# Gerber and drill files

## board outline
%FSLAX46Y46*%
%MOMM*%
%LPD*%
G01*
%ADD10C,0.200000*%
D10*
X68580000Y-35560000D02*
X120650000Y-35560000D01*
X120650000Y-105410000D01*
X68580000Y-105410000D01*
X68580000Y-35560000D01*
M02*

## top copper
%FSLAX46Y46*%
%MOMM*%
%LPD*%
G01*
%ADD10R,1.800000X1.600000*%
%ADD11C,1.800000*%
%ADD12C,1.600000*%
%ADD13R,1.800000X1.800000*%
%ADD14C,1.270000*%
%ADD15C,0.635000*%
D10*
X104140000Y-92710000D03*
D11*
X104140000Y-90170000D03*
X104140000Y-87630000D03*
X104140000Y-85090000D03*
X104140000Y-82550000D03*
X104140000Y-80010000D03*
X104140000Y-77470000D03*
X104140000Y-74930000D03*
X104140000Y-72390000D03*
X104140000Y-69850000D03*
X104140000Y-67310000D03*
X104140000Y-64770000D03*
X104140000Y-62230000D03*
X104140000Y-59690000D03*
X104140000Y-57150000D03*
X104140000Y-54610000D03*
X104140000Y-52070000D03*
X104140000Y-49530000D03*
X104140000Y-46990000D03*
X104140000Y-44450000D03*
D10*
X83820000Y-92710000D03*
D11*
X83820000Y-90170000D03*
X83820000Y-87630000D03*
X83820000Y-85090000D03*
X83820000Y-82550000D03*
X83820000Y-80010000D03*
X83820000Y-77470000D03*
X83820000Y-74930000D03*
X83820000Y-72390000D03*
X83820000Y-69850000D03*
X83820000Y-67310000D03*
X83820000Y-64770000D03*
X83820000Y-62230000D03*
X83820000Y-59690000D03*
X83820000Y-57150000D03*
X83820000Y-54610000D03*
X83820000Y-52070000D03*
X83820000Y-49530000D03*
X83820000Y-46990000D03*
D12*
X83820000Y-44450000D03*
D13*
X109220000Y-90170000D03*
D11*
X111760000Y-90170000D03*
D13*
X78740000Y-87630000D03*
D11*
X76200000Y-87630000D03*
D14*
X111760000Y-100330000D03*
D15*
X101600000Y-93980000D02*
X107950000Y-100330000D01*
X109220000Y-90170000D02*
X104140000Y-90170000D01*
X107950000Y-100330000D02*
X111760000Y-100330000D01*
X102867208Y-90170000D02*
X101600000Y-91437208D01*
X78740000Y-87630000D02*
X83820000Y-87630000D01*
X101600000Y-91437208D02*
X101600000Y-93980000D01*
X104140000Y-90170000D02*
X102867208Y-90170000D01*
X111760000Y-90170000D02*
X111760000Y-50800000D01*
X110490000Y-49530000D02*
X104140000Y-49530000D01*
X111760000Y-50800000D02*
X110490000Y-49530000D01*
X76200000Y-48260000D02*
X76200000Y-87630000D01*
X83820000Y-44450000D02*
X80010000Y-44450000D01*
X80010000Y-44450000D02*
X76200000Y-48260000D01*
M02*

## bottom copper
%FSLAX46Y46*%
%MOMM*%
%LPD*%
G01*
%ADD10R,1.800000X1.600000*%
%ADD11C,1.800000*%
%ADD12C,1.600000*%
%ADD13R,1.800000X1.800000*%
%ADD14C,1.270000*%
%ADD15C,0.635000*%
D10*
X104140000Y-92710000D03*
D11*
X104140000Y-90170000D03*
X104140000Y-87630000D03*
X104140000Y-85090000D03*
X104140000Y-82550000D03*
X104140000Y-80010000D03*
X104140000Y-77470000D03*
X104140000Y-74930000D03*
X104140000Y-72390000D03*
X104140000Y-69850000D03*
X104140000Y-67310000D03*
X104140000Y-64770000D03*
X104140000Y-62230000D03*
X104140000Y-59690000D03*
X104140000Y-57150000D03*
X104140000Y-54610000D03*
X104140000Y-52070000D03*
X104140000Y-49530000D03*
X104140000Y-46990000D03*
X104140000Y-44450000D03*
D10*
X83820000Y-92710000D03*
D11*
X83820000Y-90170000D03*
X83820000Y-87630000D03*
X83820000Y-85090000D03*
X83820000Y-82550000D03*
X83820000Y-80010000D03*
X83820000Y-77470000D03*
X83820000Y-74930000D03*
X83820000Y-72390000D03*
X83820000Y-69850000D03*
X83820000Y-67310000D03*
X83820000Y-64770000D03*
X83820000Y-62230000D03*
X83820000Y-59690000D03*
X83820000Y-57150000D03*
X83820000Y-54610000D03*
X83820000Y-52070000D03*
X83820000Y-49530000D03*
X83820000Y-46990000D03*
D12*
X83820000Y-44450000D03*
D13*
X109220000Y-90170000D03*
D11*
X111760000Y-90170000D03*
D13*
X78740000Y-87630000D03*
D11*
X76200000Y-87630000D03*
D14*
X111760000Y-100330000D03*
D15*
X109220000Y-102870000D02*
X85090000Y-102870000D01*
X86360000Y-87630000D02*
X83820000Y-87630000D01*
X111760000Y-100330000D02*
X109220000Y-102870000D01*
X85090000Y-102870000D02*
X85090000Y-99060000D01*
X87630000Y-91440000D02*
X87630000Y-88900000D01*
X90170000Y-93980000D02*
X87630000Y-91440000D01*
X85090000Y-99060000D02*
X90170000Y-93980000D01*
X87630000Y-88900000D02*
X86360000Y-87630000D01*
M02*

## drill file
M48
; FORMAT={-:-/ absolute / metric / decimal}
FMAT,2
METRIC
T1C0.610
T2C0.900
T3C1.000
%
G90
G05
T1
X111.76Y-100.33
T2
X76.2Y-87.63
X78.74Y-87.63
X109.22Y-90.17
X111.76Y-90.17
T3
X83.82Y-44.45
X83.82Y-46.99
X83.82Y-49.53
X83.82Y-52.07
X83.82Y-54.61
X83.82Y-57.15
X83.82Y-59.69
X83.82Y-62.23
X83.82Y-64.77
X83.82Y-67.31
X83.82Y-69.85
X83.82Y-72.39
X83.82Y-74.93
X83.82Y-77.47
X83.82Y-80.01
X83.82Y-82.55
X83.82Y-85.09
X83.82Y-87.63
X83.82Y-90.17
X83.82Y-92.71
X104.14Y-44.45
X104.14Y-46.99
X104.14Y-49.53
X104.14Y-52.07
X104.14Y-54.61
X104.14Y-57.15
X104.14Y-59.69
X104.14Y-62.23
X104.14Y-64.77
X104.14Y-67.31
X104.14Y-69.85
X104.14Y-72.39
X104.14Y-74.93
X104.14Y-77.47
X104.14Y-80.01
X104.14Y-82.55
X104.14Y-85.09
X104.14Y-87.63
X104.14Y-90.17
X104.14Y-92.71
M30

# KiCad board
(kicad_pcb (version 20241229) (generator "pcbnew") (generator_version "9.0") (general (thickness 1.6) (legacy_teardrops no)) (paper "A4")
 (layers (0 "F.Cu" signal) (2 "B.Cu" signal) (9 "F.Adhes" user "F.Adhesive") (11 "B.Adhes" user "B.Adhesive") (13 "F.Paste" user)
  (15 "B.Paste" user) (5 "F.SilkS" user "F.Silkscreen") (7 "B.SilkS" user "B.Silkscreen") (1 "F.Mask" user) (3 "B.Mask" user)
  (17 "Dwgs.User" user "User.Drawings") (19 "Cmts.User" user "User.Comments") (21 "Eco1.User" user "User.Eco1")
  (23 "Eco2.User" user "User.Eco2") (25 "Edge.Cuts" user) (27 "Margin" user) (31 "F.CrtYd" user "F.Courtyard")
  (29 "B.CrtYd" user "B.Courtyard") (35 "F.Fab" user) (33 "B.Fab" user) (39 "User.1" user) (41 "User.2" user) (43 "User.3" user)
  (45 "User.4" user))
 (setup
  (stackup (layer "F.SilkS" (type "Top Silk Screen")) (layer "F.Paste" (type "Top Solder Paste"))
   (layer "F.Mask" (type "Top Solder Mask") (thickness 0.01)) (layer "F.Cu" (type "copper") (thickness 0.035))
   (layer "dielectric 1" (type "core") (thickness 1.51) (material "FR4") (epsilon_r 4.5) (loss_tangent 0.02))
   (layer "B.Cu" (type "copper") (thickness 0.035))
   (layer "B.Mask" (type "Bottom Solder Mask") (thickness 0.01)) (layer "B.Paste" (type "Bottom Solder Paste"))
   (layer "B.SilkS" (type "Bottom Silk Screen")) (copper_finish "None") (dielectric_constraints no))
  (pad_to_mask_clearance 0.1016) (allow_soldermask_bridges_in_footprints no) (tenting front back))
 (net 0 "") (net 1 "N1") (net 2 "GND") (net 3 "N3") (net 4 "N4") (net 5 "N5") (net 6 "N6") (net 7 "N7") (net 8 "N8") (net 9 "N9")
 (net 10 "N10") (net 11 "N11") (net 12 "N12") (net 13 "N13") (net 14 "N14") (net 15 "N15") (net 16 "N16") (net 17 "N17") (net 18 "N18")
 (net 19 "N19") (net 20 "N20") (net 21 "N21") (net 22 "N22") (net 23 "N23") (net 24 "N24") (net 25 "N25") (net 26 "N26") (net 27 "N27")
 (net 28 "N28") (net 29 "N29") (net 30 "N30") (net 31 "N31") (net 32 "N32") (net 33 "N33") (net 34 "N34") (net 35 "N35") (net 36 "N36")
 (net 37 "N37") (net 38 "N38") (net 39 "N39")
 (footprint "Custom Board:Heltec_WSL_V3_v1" (layer "F.Cu") (at 93.98 72.39)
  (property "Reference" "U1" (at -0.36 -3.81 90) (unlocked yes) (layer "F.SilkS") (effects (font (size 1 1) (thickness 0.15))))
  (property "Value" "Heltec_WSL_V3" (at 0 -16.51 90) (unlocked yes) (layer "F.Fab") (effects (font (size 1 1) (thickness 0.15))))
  (pad "1" thru_hole rect (at 10.16 20.32) (size 1.8 1.6) (drill 1) (layers "*.Cu" "*.Mask") (remove_unused_layers no) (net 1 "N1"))
  (pad "2" thru_hole circle (at 10.16 17.78 270) (size 1.8 1.8) (drill 1) (layers "*.Cu" "*.Mask") (remove_unused_layers no) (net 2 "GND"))
  (pad "3" thru_hole circle (at 10.16 15.24 270) (size 1.8 1.8) (drill 1) (layers "*.Cu" "*.Mask") (remove_unused_layers no) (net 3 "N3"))
  (pad "4" thru_hole circle (at 10.16 12.7 270) (size 1.8 1.8) (drill 1) (layers "*.Cu" "*.Mask") (remove_unused_layers no) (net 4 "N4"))
  (pad "5" thru_hole circle (at 10.16 10.16 270) (size 1.8 1.8) (drill 1) (layers "*.Cu" "*.Mask") (remove_unused_layers no) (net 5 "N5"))
  (pad "6" thru_hole circle (at 10.16 7.62 270) (size 1.8 1.8) (drill 1) (layers "*.Cu" "*.Mask") (remove_unused_layers no) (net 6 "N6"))
  (pad "7" thru_hole circle (at 10.16 5.08 270) (size 1.8 1.8) (drill 1) (layers "*.Cu" "*.Mask") (remove_unused_layers no) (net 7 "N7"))
  (pad "8" thru_hole circle (at 10.16 2.54 270) (size 1.8 1.8) (drill 1) (layers "*.Cu" "*.Mask") (remove_unused_layers no) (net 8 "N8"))
  (pad "9" thru_hole circle (at 10.16 0 270) (size 1.8 1.8) (drill 1) (layers "*.Cu" "*.Mask") (remove_unused_layers no) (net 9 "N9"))
  (pad "10" thru_hole circle (at 10.16 -2.54 270) (size 1.8 1.8) (drill 1) (layers "*.Cu" "*.Mask") (remove_unused_layers no) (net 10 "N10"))
  (pad "11" thru_hole circle (at 10.16 -5.08 270) (size 1.8 1.8) (drill 1) (layers "*.Cu" "*.Mask") (remove_unused_layers no) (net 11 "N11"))
  (pad "12" thru_hole circle (at 10.16 -7.62 270) (size 1.8 1.8) (drill 1) (layers "*.Cu" "*.Mask") (remove_unused_layers no) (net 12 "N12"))
  (pad "13" thru_hole circle (at 10.16 -10.16 270) (size 1.8 1.8) (drill 1) (layers "*.Cu" "*.Mask") (remove_unused_layers no)
   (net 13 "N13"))
  (pad "14" thru_hole circle (at 10.16 -12.7 270) (size 1.8 1.8) (drill 1) (layers "*.Cu" "*.Mask") (remove_unused_layers no) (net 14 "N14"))
  (pad "15" thru_hole circle (at 10.16 -15.24 270) (size 1.8 1.8) (drill 1) (layers "*.Cu" "*.Mask") (remove_unused_layers no)
   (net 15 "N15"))
  (pad "16" thru_hole circle (at 10.16 -17.78 270) (size 1.8 1.8) (drill 1) (layers "*.Cu" "*.Mask") (remove_unused_layers no)
   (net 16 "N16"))
  (pad "17" thru_hole circle (at 10.16 -20.32 270) (size 1.8 1.8) (drill 1) (layers "*.Cu" "*.Mask") (remove_unused_layers no)
   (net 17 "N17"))
  (pad "18" thru_hole circle (at 10.16 -22.86 270) (size 1.8 1.8) (drill 1) (layers "*.Cu" "*.Mask") (remove_unused_layers no)
   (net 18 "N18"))
  (pad "19" thru_hole circle (at 10.16 -25.4 270) (size 1.8 1.8) (drill 1) (layers "*.Cu" "*.Mask") (remove_unused_layers no) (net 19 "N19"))
  (pad "20" thru_hole circle (at 10.16 -27.94 270) (size 1.8 1.8) (drill 1) (layers "*.Cu" "*.Mask") (remove_unused_layers no)
   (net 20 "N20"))
  (pad "21" thru_hole rect (at -10.16 20.32) (size 1.8 1.6) (drill 1) (layers "*.Cu" "*.Mask") (remove_unused_layers no) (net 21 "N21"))
  (pad "22" thru_hole circle (at -10.16 17.78 270) (size 1.8 1.8) (drill 1) (layers "*.Cu" "*.Mask") (remove_unused_layers no)
   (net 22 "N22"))
  (pad "23" thru_hole circle (at -10.16 15.24 270) (size 1.8 1.8) (drill 1) (layers "*.Cu" "*.Mask") (remove_unused_layers no) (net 2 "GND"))
  (pad "24" thru_hole circle (at -10.16 12.7 270) (size 1.8 1.8) (drill 1) (layers "*.Cu" "*.Mask") (remove_unused_layers no) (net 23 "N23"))
  (pad "25" thru_hole circle (at -10.16 10.16 270) (size 1.8 1.8) (drill 1) (layers "*.Cu" "*.Mask") (remove_unused_layers no)
   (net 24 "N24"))
  (pad "26" thru_hole circle (at -10.16 7.62 270) (size 1.8 1.8) (drill 1) (layers "*.Cu" "*.Mask") (remove_unused_layers no) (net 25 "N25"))
  (pad "27" thru_hole circle (at -10.16 5.08 270) (size 1.8 1.8) (drill 1) (layers "*.Cu" "*.Mask") (remove_unused_layers no) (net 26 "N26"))
  (pad "28" thru_hole circle (at -10.16 2.54 270) (size 1.8 1.8) (drill 1) (layers "*.Cu" "*.Mask") (remove_unused_layers no) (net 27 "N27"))
  (pad "29" thru_hole circle (at -10.16 0 270) (size 1.8 1.8) (drill 1) (layers "*.Cu" "*.Mask") (remove_unused_layers no) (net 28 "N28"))
  (pad "30" thru_hole circle (at -10.16 -2.54 270) (size 1.8 1.8) (drill 1) (layers "*.Cu" "*.Mask") (remove_unused_layers no)
   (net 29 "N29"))
  (pad "31" thru_hole circle (at -10.16 -5.08 270) (size 1.8 1.8) (drill 1) (layers "*.Cu" "*.Mask") (remove_unused_layers no)
   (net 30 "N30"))
  (pad "32" thru_hole circle (at -10.16 -7.62 270) (size 1.8 1.8) (drill 1) (layers "*.Cu" "*.Mask") (remove_unused_layers no)
   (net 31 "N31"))
  (pad "33" thru_hole circle (at -10.16 -10.16 270) (size 1.8 1.8) (drill 1) (layers "*.Cu" "*.Mask") (remove_unused_layers no)
   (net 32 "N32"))
  (pad "34" thru_hole circle (at -10.16 -12.7 270) (size 1.8 1.8) (drill 1) (layers "*.Cu" "*.Mask") (remove_unused_layers no)
   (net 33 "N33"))
  (pad "35" thru_hole circle (at -10.16 -15.24 270) (size 1.8 1.8) (drill 1) (layers "*.Cu" "*.Mask") (remove_unused_layers no)
   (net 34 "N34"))
  (pad "36" thru_hole circle (at -10.16 -17.78 270) (size 1.8 1.8) (drill 1) (layers "*.Cu" "*.Mask") (remove_unused_layers no)
   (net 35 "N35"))
  (pad "37" thru_hole circle (at -10.16 -20.32 270) (size 1.8 1.8) (drill 1) (layers "*.Cu" "*.Mask") (remove_unused_layers no)
   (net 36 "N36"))
  (pad "38" thru_hole circle (at -10.16 -22.86 270) (size 1.8 1.8) (drill 1) (layers "*.Cu" "*.Mask") (remove_unused_layers no)
   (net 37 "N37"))
  (pad "39" thru_hole circle (at -10.16 -25.4 270) (size 1.8 1.8) (drill 1) (layers "*.Cu" "*.Mask") (remove_unused_layers no)
   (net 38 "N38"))
  (pad "40" thru_hole circle (at -10.16 -27.94 270) (size 1.6 1.6) (drill 1) (layers "*.Cu" "*.Mask") (remove_unused_layers no)
   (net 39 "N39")))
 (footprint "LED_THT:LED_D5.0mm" (layer "F.Cu") (at 109.22 90.17)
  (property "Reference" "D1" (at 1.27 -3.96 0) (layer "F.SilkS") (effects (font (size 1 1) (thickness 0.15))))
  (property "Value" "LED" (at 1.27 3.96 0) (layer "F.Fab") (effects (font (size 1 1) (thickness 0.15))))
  (pad "1" thru_hole rect (at 0 0) (size 1.8 1.8) (drill 0.9) (layers "*.Cu" "*.Mask") (remove_unused_layers no) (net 2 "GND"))
  (pad "2" thru_hole circle (at 2.54 0) (size 1.8 1.8) (drill 0.9) (layers "*.Cu" "*.Mask") (remove_unused_layers no) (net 18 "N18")))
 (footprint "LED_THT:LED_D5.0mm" (layer "F.Cu") (at 78.74 87.63 180)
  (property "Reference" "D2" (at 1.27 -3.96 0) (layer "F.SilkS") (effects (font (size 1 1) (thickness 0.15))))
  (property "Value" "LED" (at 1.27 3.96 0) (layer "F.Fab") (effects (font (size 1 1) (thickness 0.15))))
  (pad "1" thru_hole rect (at 0 0 180) (size 1.8 1.8) (drill 0.9) (layers "*.Cu" "*.Mask") (remove_unused_layers no) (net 2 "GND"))
  (pad "2" thru_hole circle (at 2.54 0 180) (size 1.8 1.8) (drill 0.9) (layers "*.Cu" "*.Mask") (remove_unused_layers no) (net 39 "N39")))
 (gr_rect (start 68.58 35.56) (end 120.65 105.41) (stroke (width 0.2) (type default)) (fill no) (layer "Edge.Cuts"))
 (segment (start 101.6 93.98) (end 107.95 100.33) (width 0.635) (layer "F.Cu") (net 2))
 (segment (start 109.22 90.17) (end 104.14 90.17) (width 0.635) (layer "F.Cu") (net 2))
 (segment (start 107.95 100.33) (end 111.76 100.33) (width 0.635) (layer "F.Cu") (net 2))
 (segment (start 102.867208 90.17) (end 101.6 91.437208) (width 0.635) (layer "F.Cu") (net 2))
 (segment (start 78.74 87.63) (end 83.82 87.63) (width 0.635) (layer "F.Cu") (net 2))
 (segment (start 101.6 91.437208) (end 101.6 93.98) (width 0.635) (layer "F.Cu") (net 2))
 (segment (start 104.14 90.17) (end 102.867208 90.17) (width 0.635) (layer "F.Cu") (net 2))
 (via (at 111.76 100.33) (size 1.27) (drill 0.6096) (layers "F.Cu" "B.Cu") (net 2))
 (segment (start 109.22 102.87) (end 85.09 102.87) (width 0.635) (layer "B.Cu") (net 2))
 (segment (start 86.36 87.63) (end 83.82 87.63) (width 0.635) (layer "B.Cu") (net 2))
 (segment (start 111.76 100.33) (end 109.22 102.87) (width 0.635) (layer "B.Cu") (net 2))
 (segment (start 85.09 102.87) (end 85.09 99.06) (width 0.635) (layer "B.Cu") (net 2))
 (segment (start 87.63 91.44) (end 87.63 88.9) (width 0.635) (layer "B.Cu") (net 2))
 (segment (start 90.17 93.98) (end 87.63 91.44) (width 0.635) (layer "B.Cu") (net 2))
 (segment (start 85.09 99.06) (end 90.17 93.98) (width 0.635) (layer "B.Cu") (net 2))
 (segment (start 87.63 88.9) (end 86.36 87.63) (width 0.635) (layer "B.Cu") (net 2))
 (segment (start 111.76 90.17) (end 111.76 50.8) (width 0.635) (layer "F.Cu") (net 18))
 (segment (start 110.49 49.53) (end 104.14 49.53) (width 0.635) (layer "F.Cu") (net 18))
 (segment (start 111.76 50.8) (end 110.49 49.53) (width 0.635) (layer "F.Cu") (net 18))
 (segment (start 76.2 48.26) (end 76.2 87.63) (width 0.635) (layer "F.Cu") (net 39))
 (segment (start 83.82 44.45) (end 80.01 44.45) (width 0.635) (layer "F.Cu") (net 39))
 (segment (start 80.01 44.45) (end 76.2 48.26) (width 0.635) (layer "F.Cu") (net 39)))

